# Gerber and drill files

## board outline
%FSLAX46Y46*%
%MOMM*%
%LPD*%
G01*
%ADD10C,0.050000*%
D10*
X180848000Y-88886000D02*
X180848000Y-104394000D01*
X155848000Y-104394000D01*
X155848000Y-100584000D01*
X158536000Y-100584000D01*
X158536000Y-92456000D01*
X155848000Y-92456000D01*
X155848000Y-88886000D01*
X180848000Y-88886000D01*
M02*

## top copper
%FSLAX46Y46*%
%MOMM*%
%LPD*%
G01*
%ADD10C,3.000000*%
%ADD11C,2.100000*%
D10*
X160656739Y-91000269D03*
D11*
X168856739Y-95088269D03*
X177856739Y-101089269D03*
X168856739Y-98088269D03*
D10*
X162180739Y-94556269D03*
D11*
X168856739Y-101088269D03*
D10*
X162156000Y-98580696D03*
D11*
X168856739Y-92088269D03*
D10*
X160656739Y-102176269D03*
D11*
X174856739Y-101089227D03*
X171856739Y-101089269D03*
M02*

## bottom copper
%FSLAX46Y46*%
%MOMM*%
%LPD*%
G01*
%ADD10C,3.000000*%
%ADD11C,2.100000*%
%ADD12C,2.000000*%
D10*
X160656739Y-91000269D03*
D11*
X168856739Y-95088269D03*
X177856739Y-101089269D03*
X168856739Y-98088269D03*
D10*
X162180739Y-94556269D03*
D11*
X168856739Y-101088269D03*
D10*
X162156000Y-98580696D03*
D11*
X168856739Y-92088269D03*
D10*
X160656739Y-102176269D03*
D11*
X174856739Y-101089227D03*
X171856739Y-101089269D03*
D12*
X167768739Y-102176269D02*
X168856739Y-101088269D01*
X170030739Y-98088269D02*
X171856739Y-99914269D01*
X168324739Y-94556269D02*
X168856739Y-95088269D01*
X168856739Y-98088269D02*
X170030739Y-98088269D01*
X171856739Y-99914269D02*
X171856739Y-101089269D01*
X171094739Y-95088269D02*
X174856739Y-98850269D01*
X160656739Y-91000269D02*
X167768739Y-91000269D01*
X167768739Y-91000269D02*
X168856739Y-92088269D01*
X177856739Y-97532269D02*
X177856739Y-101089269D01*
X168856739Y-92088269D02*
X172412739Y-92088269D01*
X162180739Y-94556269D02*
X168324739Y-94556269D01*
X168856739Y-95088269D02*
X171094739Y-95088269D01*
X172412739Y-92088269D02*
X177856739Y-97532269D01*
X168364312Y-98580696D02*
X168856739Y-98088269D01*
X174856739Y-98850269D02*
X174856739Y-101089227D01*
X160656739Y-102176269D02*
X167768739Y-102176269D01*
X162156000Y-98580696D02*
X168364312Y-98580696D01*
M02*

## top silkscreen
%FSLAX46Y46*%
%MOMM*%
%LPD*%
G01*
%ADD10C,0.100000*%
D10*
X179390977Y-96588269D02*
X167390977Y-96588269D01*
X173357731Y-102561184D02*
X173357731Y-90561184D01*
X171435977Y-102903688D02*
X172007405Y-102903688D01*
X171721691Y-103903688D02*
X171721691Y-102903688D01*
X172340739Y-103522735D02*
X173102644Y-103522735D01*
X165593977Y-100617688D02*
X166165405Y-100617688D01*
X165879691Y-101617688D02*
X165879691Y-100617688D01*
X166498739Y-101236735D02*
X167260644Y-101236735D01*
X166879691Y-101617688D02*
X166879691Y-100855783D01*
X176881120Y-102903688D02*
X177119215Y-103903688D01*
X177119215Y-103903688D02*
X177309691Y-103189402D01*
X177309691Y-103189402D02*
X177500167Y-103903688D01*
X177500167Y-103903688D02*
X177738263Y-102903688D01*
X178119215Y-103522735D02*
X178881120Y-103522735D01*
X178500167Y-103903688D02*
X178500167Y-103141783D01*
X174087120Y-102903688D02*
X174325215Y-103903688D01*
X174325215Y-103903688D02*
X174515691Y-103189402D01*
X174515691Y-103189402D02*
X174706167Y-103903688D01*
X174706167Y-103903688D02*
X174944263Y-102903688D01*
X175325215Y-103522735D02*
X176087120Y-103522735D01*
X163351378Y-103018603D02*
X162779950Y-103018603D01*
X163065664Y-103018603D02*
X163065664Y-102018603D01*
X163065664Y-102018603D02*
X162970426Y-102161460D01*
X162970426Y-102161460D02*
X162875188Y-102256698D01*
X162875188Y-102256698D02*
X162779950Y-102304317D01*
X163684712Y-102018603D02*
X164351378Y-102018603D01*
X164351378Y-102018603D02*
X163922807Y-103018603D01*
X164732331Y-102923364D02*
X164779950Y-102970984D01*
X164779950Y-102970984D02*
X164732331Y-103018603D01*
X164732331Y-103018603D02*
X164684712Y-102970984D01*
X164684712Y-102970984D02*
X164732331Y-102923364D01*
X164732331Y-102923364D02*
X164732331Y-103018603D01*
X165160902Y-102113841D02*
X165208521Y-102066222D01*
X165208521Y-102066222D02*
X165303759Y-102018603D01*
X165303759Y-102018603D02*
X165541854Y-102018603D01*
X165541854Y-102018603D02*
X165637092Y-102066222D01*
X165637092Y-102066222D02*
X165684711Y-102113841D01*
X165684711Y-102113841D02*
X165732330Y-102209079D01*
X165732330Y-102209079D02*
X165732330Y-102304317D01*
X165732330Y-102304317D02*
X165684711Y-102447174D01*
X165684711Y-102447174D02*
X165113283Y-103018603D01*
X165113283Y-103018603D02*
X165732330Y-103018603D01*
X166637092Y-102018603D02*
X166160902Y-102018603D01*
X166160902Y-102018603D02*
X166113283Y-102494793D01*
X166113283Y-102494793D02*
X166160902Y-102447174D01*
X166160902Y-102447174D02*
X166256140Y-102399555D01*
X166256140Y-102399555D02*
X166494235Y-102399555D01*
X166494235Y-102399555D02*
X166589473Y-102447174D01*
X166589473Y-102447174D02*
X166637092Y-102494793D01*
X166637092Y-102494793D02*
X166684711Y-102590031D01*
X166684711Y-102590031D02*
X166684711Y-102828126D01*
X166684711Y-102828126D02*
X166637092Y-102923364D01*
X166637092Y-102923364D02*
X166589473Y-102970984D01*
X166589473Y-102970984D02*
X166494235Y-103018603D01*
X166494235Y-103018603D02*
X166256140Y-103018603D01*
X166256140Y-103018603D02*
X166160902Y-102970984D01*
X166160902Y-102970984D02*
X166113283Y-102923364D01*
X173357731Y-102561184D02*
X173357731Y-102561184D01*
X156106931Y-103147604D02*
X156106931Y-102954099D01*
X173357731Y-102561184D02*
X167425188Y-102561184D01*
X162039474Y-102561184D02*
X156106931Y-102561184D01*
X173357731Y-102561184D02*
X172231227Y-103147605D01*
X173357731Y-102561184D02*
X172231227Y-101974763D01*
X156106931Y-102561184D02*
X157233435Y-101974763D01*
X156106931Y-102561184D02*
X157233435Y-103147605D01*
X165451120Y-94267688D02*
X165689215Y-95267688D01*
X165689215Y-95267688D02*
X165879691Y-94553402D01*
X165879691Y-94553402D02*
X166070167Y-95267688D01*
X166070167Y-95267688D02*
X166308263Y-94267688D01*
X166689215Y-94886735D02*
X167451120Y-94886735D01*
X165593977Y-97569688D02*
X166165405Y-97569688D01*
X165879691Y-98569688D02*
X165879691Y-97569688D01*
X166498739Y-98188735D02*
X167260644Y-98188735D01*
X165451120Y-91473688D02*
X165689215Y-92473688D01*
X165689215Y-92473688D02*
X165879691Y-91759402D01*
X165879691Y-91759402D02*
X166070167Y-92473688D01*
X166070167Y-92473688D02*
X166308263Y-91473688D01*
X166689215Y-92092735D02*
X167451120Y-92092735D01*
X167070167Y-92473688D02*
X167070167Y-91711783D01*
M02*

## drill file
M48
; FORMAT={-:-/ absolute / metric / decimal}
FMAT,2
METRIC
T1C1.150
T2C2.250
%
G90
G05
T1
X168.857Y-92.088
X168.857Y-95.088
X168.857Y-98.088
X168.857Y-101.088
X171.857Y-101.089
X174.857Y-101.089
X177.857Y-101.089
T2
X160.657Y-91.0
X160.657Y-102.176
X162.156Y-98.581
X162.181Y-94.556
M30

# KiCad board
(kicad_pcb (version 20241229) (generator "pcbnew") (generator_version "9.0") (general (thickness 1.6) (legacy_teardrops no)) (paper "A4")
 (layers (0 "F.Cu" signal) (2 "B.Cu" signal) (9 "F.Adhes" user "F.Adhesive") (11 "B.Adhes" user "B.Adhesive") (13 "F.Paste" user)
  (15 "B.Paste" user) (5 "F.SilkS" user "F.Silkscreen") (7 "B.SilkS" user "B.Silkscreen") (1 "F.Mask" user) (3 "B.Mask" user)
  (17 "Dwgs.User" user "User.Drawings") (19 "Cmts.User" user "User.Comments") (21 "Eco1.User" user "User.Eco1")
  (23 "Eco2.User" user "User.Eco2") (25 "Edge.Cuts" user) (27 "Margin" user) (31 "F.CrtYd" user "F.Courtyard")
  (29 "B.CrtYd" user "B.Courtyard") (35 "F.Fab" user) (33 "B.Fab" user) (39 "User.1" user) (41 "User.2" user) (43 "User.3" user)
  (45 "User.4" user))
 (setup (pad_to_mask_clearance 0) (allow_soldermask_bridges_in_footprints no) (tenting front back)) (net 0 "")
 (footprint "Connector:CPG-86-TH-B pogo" (layer "F.Cu") (at 160.656739 91.000269)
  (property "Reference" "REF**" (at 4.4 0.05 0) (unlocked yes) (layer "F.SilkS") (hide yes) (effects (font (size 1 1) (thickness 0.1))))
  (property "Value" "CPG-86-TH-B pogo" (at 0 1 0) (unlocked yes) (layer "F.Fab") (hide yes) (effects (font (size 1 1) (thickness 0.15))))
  (pad "1" thru_hole circle (at 0 0) (size 3 3) (drill 2.25) (layers "*.Cu" "*.Mask") (remove_unused_layers no)))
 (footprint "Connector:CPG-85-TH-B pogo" (layer "F.Cu") (at 168.856739 95.088269)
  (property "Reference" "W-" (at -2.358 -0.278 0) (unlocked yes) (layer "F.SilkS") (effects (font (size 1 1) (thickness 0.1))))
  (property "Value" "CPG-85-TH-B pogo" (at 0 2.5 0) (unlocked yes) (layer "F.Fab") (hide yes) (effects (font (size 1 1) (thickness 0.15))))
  (pad "1" thru_hole circle (at 0 0) (size 2.1 2.1) (drill 1.15) (layers "*.Cu" "*.Mask") (remove_unused_layers no)))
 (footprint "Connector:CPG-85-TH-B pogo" (layer "F.Cu") (at 177.856739 101.089269)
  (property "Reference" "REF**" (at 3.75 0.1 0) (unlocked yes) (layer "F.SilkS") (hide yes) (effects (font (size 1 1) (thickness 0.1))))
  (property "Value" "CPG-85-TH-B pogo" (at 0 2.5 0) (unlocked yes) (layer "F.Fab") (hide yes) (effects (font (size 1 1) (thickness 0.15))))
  (pad "1" thru_hole circle (at 0 0) (size 2.1 2.1) (drill 1.15) (layers "*.Cu" "*.Mask") (remove_unused_layers no)))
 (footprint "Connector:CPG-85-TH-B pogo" (layer "F.Cu") (at 168.856739 98.088269)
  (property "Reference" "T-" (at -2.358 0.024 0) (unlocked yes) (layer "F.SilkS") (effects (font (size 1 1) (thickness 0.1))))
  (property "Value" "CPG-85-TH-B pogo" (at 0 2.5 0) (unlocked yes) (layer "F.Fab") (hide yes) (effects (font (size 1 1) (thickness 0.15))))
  (pad "1" thru_hole circle (at 0 0) (size 2.1 2.1) (drill 1.15) (layers "*.Cu" "*.Mask") (remove_unused_layers no)))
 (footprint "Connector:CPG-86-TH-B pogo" (layer "F.Cu") (at 162.180739 94.556269)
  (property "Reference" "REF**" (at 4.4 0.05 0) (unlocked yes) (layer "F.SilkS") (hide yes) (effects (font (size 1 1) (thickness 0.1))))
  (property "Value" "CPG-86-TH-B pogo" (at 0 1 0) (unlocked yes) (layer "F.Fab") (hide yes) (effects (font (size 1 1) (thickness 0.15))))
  (pad "1" thru_hole circle (at 0 0) (size 3 3) (drill 2.25) (layers "*.Cu" "*.Mask") (remove_unused_layers no)))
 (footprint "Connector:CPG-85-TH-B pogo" (layer "F.Cu") (at 168.856739 101.088269)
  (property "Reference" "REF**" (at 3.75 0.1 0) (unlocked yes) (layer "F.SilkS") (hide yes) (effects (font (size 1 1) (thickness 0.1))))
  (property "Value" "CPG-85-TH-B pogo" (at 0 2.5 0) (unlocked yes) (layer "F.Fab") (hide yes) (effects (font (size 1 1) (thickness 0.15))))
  (pad "1" thru_hole circle (at 0 0) (size 2.1 2.1) (drill 1.15) (layers "*.Cu" "*.Mask") (remove_unused_layers no)))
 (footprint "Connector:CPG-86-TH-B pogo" (layer "F.Cu") (at 162.156 98.580696)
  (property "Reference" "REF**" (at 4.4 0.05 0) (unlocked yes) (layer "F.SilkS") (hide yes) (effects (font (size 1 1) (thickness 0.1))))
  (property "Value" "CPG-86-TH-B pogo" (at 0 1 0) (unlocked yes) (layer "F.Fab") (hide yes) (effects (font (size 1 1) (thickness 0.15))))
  (pad "1" thru_hole circle (at 0 0) (size 3 3) (drill 2.25) (layers "*.Cu" "*.Mask") (remove_unused_layers no)))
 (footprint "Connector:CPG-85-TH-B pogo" (layer "F.Cu") (at 168.856739 92.088269)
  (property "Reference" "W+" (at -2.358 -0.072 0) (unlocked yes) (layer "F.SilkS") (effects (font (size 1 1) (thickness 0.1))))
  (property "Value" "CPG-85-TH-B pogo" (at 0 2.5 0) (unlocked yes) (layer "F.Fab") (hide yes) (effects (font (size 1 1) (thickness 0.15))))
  (pad "1" thru_hole circle (at 0 0) (size 2.1 2.1) (drill 1.15) (layers "*.Cu" "*.Mask") (remove_unused_layers no)))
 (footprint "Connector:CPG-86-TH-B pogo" (layer "F.Cu") (at 160.656739 102.176269)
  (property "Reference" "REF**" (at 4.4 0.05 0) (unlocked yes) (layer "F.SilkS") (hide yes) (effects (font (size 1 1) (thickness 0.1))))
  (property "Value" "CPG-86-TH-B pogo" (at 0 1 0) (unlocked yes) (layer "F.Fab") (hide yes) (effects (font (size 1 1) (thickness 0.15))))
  (pad "1" thru_hole circle (at 0 0) (size 3 3) (drill 2.25) (layers "*.Cu" "*.Mask") (remove_unused_layers no)))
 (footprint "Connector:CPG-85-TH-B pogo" (layer "F.Cu") (at 174.856739 101.089227)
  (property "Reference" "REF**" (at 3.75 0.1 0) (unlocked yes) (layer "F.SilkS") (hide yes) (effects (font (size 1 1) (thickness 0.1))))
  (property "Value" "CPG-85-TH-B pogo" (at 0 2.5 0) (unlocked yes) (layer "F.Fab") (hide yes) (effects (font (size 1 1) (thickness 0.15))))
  (pad "1" thru_hole circle (at 0 0) (size 2.1 2.1) (drill 1.15) (layers "*.Cu" "*.Mask") (remove_unused_layers no)))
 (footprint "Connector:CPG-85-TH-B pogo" (layer "F.Cu") (at 171.856739 101.089269)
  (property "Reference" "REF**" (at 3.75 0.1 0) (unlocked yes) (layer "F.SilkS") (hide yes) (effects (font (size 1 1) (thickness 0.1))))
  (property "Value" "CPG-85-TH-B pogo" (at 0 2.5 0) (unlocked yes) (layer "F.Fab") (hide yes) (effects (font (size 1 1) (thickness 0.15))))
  (pad "1" thru_hole circle (at 0 0) (size 2.1 2.1) (drill 1.15) (layers "*.Cu" "*.Mask") (remove_unused_layers no)))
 (gr_line (start 179.390977 96.588269) (end 167.390977 96.588269) (stroke (width 0.1) (type solid)) (layer "F.SilkS"))
 (gr_line (start 173.357731 102.561184) (end 173.357731 90.561184) (stroke (width 0.1) (type solid)) (layer "F.SilkS"))
 (gr_poly
  (pts (xy 180.848 88.886) (xy 180.848 104.394) (xy 155.848 104.394) (xy 155.848 100.584) (xy 158.536 100.584) (xy 158.536 92.456)
   (xy 155.848 92.456) (xy 155.848 88.886))
  (stroke (width 0.05) (type solid)) (fill no) (layer "Edge.Cuts"))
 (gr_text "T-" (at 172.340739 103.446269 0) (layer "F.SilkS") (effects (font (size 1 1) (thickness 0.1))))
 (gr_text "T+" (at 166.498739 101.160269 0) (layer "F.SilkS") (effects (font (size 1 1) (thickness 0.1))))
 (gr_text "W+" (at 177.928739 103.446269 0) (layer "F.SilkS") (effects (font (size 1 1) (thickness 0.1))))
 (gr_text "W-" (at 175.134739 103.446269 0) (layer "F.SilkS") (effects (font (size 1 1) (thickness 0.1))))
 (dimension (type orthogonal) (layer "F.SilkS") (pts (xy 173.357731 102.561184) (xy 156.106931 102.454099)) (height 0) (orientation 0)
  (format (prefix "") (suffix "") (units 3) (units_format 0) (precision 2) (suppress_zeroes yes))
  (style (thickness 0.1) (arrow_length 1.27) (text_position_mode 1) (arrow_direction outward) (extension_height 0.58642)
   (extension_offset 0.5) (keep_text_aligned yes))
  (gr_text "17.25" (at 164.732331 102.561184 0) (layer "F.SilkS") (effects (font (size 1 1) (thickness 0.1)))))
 (segment (start 167.768739 102.176269) (end 168.856739 101.088269) (width 2) (layer "B.Cu") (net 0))
 (segment (start 170.030739 98.088269) (end 171.856739 99.914269) (width 2) (layer "B.Cu") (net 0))
 (segment (start 168.324739 94.556269) (end 168.856739 95.088269) (width 2) (layer "B.Cu") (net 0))
 (segment (start 168.856739 98.088269) (end 170.030739 98.088269) (width 2) (layer "B.Cu") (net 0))
 (segment (start 171.856739 99.914269) (end 171.856739 101.089269) (width 2) (layer "B.Cu") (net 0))
 (segment (start 171.094739 95.088269) (end 174.856739 98.850269) (width 2) (layer "B.Cu") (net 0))
 (segment (start 160.656739 91.000269) (end 167.768739 91.000269) (width 2) (layer "B.Cu") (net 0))
 (segment (start 167.768739 91.000269) (end 168.856739 92.088269) (width 2) (layer "B.Cu") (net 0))
 (segment (start 177.856739 97.532269) (end 177.856739 101.089269) (width 2) (layer "B.Cu") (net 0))
 (segment (start 168.856739 92.088269) (end 172.412739 92.088269) (width 2) (layer "B.Cu") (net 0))
 (segment (start 162.180739 94.556269) (end 168.324739 94.556269) (width 2) (layer "B.Cu") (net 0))
 (segment (start 168.856739 95.088269) (end 171.094739 95.088269) (width 2) (layer "B.Cu") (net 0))
 (segment (start 172.412739 92.088269) (end 177.856739 97.532269) (width 2) (layer "B.Cu") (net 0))
 (segment (start 168.364312 98.580696) (end 168.856739 98.088269) (width 2) (layer "B.Cu") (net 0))
 (segment (start 174.856739 98.850269) (end 174.856739 101.089227) (width 2) (layer "B.Cu") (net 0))
 (segment (start 160.656739 102.176269) (end 167.768739 102.176269) (width 2) (layer "B.Cu") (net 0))
 (segment (start 162.156 98.580696) (end 168.364312 98.580696) (width 2) (layer "B.Cu") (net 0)))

